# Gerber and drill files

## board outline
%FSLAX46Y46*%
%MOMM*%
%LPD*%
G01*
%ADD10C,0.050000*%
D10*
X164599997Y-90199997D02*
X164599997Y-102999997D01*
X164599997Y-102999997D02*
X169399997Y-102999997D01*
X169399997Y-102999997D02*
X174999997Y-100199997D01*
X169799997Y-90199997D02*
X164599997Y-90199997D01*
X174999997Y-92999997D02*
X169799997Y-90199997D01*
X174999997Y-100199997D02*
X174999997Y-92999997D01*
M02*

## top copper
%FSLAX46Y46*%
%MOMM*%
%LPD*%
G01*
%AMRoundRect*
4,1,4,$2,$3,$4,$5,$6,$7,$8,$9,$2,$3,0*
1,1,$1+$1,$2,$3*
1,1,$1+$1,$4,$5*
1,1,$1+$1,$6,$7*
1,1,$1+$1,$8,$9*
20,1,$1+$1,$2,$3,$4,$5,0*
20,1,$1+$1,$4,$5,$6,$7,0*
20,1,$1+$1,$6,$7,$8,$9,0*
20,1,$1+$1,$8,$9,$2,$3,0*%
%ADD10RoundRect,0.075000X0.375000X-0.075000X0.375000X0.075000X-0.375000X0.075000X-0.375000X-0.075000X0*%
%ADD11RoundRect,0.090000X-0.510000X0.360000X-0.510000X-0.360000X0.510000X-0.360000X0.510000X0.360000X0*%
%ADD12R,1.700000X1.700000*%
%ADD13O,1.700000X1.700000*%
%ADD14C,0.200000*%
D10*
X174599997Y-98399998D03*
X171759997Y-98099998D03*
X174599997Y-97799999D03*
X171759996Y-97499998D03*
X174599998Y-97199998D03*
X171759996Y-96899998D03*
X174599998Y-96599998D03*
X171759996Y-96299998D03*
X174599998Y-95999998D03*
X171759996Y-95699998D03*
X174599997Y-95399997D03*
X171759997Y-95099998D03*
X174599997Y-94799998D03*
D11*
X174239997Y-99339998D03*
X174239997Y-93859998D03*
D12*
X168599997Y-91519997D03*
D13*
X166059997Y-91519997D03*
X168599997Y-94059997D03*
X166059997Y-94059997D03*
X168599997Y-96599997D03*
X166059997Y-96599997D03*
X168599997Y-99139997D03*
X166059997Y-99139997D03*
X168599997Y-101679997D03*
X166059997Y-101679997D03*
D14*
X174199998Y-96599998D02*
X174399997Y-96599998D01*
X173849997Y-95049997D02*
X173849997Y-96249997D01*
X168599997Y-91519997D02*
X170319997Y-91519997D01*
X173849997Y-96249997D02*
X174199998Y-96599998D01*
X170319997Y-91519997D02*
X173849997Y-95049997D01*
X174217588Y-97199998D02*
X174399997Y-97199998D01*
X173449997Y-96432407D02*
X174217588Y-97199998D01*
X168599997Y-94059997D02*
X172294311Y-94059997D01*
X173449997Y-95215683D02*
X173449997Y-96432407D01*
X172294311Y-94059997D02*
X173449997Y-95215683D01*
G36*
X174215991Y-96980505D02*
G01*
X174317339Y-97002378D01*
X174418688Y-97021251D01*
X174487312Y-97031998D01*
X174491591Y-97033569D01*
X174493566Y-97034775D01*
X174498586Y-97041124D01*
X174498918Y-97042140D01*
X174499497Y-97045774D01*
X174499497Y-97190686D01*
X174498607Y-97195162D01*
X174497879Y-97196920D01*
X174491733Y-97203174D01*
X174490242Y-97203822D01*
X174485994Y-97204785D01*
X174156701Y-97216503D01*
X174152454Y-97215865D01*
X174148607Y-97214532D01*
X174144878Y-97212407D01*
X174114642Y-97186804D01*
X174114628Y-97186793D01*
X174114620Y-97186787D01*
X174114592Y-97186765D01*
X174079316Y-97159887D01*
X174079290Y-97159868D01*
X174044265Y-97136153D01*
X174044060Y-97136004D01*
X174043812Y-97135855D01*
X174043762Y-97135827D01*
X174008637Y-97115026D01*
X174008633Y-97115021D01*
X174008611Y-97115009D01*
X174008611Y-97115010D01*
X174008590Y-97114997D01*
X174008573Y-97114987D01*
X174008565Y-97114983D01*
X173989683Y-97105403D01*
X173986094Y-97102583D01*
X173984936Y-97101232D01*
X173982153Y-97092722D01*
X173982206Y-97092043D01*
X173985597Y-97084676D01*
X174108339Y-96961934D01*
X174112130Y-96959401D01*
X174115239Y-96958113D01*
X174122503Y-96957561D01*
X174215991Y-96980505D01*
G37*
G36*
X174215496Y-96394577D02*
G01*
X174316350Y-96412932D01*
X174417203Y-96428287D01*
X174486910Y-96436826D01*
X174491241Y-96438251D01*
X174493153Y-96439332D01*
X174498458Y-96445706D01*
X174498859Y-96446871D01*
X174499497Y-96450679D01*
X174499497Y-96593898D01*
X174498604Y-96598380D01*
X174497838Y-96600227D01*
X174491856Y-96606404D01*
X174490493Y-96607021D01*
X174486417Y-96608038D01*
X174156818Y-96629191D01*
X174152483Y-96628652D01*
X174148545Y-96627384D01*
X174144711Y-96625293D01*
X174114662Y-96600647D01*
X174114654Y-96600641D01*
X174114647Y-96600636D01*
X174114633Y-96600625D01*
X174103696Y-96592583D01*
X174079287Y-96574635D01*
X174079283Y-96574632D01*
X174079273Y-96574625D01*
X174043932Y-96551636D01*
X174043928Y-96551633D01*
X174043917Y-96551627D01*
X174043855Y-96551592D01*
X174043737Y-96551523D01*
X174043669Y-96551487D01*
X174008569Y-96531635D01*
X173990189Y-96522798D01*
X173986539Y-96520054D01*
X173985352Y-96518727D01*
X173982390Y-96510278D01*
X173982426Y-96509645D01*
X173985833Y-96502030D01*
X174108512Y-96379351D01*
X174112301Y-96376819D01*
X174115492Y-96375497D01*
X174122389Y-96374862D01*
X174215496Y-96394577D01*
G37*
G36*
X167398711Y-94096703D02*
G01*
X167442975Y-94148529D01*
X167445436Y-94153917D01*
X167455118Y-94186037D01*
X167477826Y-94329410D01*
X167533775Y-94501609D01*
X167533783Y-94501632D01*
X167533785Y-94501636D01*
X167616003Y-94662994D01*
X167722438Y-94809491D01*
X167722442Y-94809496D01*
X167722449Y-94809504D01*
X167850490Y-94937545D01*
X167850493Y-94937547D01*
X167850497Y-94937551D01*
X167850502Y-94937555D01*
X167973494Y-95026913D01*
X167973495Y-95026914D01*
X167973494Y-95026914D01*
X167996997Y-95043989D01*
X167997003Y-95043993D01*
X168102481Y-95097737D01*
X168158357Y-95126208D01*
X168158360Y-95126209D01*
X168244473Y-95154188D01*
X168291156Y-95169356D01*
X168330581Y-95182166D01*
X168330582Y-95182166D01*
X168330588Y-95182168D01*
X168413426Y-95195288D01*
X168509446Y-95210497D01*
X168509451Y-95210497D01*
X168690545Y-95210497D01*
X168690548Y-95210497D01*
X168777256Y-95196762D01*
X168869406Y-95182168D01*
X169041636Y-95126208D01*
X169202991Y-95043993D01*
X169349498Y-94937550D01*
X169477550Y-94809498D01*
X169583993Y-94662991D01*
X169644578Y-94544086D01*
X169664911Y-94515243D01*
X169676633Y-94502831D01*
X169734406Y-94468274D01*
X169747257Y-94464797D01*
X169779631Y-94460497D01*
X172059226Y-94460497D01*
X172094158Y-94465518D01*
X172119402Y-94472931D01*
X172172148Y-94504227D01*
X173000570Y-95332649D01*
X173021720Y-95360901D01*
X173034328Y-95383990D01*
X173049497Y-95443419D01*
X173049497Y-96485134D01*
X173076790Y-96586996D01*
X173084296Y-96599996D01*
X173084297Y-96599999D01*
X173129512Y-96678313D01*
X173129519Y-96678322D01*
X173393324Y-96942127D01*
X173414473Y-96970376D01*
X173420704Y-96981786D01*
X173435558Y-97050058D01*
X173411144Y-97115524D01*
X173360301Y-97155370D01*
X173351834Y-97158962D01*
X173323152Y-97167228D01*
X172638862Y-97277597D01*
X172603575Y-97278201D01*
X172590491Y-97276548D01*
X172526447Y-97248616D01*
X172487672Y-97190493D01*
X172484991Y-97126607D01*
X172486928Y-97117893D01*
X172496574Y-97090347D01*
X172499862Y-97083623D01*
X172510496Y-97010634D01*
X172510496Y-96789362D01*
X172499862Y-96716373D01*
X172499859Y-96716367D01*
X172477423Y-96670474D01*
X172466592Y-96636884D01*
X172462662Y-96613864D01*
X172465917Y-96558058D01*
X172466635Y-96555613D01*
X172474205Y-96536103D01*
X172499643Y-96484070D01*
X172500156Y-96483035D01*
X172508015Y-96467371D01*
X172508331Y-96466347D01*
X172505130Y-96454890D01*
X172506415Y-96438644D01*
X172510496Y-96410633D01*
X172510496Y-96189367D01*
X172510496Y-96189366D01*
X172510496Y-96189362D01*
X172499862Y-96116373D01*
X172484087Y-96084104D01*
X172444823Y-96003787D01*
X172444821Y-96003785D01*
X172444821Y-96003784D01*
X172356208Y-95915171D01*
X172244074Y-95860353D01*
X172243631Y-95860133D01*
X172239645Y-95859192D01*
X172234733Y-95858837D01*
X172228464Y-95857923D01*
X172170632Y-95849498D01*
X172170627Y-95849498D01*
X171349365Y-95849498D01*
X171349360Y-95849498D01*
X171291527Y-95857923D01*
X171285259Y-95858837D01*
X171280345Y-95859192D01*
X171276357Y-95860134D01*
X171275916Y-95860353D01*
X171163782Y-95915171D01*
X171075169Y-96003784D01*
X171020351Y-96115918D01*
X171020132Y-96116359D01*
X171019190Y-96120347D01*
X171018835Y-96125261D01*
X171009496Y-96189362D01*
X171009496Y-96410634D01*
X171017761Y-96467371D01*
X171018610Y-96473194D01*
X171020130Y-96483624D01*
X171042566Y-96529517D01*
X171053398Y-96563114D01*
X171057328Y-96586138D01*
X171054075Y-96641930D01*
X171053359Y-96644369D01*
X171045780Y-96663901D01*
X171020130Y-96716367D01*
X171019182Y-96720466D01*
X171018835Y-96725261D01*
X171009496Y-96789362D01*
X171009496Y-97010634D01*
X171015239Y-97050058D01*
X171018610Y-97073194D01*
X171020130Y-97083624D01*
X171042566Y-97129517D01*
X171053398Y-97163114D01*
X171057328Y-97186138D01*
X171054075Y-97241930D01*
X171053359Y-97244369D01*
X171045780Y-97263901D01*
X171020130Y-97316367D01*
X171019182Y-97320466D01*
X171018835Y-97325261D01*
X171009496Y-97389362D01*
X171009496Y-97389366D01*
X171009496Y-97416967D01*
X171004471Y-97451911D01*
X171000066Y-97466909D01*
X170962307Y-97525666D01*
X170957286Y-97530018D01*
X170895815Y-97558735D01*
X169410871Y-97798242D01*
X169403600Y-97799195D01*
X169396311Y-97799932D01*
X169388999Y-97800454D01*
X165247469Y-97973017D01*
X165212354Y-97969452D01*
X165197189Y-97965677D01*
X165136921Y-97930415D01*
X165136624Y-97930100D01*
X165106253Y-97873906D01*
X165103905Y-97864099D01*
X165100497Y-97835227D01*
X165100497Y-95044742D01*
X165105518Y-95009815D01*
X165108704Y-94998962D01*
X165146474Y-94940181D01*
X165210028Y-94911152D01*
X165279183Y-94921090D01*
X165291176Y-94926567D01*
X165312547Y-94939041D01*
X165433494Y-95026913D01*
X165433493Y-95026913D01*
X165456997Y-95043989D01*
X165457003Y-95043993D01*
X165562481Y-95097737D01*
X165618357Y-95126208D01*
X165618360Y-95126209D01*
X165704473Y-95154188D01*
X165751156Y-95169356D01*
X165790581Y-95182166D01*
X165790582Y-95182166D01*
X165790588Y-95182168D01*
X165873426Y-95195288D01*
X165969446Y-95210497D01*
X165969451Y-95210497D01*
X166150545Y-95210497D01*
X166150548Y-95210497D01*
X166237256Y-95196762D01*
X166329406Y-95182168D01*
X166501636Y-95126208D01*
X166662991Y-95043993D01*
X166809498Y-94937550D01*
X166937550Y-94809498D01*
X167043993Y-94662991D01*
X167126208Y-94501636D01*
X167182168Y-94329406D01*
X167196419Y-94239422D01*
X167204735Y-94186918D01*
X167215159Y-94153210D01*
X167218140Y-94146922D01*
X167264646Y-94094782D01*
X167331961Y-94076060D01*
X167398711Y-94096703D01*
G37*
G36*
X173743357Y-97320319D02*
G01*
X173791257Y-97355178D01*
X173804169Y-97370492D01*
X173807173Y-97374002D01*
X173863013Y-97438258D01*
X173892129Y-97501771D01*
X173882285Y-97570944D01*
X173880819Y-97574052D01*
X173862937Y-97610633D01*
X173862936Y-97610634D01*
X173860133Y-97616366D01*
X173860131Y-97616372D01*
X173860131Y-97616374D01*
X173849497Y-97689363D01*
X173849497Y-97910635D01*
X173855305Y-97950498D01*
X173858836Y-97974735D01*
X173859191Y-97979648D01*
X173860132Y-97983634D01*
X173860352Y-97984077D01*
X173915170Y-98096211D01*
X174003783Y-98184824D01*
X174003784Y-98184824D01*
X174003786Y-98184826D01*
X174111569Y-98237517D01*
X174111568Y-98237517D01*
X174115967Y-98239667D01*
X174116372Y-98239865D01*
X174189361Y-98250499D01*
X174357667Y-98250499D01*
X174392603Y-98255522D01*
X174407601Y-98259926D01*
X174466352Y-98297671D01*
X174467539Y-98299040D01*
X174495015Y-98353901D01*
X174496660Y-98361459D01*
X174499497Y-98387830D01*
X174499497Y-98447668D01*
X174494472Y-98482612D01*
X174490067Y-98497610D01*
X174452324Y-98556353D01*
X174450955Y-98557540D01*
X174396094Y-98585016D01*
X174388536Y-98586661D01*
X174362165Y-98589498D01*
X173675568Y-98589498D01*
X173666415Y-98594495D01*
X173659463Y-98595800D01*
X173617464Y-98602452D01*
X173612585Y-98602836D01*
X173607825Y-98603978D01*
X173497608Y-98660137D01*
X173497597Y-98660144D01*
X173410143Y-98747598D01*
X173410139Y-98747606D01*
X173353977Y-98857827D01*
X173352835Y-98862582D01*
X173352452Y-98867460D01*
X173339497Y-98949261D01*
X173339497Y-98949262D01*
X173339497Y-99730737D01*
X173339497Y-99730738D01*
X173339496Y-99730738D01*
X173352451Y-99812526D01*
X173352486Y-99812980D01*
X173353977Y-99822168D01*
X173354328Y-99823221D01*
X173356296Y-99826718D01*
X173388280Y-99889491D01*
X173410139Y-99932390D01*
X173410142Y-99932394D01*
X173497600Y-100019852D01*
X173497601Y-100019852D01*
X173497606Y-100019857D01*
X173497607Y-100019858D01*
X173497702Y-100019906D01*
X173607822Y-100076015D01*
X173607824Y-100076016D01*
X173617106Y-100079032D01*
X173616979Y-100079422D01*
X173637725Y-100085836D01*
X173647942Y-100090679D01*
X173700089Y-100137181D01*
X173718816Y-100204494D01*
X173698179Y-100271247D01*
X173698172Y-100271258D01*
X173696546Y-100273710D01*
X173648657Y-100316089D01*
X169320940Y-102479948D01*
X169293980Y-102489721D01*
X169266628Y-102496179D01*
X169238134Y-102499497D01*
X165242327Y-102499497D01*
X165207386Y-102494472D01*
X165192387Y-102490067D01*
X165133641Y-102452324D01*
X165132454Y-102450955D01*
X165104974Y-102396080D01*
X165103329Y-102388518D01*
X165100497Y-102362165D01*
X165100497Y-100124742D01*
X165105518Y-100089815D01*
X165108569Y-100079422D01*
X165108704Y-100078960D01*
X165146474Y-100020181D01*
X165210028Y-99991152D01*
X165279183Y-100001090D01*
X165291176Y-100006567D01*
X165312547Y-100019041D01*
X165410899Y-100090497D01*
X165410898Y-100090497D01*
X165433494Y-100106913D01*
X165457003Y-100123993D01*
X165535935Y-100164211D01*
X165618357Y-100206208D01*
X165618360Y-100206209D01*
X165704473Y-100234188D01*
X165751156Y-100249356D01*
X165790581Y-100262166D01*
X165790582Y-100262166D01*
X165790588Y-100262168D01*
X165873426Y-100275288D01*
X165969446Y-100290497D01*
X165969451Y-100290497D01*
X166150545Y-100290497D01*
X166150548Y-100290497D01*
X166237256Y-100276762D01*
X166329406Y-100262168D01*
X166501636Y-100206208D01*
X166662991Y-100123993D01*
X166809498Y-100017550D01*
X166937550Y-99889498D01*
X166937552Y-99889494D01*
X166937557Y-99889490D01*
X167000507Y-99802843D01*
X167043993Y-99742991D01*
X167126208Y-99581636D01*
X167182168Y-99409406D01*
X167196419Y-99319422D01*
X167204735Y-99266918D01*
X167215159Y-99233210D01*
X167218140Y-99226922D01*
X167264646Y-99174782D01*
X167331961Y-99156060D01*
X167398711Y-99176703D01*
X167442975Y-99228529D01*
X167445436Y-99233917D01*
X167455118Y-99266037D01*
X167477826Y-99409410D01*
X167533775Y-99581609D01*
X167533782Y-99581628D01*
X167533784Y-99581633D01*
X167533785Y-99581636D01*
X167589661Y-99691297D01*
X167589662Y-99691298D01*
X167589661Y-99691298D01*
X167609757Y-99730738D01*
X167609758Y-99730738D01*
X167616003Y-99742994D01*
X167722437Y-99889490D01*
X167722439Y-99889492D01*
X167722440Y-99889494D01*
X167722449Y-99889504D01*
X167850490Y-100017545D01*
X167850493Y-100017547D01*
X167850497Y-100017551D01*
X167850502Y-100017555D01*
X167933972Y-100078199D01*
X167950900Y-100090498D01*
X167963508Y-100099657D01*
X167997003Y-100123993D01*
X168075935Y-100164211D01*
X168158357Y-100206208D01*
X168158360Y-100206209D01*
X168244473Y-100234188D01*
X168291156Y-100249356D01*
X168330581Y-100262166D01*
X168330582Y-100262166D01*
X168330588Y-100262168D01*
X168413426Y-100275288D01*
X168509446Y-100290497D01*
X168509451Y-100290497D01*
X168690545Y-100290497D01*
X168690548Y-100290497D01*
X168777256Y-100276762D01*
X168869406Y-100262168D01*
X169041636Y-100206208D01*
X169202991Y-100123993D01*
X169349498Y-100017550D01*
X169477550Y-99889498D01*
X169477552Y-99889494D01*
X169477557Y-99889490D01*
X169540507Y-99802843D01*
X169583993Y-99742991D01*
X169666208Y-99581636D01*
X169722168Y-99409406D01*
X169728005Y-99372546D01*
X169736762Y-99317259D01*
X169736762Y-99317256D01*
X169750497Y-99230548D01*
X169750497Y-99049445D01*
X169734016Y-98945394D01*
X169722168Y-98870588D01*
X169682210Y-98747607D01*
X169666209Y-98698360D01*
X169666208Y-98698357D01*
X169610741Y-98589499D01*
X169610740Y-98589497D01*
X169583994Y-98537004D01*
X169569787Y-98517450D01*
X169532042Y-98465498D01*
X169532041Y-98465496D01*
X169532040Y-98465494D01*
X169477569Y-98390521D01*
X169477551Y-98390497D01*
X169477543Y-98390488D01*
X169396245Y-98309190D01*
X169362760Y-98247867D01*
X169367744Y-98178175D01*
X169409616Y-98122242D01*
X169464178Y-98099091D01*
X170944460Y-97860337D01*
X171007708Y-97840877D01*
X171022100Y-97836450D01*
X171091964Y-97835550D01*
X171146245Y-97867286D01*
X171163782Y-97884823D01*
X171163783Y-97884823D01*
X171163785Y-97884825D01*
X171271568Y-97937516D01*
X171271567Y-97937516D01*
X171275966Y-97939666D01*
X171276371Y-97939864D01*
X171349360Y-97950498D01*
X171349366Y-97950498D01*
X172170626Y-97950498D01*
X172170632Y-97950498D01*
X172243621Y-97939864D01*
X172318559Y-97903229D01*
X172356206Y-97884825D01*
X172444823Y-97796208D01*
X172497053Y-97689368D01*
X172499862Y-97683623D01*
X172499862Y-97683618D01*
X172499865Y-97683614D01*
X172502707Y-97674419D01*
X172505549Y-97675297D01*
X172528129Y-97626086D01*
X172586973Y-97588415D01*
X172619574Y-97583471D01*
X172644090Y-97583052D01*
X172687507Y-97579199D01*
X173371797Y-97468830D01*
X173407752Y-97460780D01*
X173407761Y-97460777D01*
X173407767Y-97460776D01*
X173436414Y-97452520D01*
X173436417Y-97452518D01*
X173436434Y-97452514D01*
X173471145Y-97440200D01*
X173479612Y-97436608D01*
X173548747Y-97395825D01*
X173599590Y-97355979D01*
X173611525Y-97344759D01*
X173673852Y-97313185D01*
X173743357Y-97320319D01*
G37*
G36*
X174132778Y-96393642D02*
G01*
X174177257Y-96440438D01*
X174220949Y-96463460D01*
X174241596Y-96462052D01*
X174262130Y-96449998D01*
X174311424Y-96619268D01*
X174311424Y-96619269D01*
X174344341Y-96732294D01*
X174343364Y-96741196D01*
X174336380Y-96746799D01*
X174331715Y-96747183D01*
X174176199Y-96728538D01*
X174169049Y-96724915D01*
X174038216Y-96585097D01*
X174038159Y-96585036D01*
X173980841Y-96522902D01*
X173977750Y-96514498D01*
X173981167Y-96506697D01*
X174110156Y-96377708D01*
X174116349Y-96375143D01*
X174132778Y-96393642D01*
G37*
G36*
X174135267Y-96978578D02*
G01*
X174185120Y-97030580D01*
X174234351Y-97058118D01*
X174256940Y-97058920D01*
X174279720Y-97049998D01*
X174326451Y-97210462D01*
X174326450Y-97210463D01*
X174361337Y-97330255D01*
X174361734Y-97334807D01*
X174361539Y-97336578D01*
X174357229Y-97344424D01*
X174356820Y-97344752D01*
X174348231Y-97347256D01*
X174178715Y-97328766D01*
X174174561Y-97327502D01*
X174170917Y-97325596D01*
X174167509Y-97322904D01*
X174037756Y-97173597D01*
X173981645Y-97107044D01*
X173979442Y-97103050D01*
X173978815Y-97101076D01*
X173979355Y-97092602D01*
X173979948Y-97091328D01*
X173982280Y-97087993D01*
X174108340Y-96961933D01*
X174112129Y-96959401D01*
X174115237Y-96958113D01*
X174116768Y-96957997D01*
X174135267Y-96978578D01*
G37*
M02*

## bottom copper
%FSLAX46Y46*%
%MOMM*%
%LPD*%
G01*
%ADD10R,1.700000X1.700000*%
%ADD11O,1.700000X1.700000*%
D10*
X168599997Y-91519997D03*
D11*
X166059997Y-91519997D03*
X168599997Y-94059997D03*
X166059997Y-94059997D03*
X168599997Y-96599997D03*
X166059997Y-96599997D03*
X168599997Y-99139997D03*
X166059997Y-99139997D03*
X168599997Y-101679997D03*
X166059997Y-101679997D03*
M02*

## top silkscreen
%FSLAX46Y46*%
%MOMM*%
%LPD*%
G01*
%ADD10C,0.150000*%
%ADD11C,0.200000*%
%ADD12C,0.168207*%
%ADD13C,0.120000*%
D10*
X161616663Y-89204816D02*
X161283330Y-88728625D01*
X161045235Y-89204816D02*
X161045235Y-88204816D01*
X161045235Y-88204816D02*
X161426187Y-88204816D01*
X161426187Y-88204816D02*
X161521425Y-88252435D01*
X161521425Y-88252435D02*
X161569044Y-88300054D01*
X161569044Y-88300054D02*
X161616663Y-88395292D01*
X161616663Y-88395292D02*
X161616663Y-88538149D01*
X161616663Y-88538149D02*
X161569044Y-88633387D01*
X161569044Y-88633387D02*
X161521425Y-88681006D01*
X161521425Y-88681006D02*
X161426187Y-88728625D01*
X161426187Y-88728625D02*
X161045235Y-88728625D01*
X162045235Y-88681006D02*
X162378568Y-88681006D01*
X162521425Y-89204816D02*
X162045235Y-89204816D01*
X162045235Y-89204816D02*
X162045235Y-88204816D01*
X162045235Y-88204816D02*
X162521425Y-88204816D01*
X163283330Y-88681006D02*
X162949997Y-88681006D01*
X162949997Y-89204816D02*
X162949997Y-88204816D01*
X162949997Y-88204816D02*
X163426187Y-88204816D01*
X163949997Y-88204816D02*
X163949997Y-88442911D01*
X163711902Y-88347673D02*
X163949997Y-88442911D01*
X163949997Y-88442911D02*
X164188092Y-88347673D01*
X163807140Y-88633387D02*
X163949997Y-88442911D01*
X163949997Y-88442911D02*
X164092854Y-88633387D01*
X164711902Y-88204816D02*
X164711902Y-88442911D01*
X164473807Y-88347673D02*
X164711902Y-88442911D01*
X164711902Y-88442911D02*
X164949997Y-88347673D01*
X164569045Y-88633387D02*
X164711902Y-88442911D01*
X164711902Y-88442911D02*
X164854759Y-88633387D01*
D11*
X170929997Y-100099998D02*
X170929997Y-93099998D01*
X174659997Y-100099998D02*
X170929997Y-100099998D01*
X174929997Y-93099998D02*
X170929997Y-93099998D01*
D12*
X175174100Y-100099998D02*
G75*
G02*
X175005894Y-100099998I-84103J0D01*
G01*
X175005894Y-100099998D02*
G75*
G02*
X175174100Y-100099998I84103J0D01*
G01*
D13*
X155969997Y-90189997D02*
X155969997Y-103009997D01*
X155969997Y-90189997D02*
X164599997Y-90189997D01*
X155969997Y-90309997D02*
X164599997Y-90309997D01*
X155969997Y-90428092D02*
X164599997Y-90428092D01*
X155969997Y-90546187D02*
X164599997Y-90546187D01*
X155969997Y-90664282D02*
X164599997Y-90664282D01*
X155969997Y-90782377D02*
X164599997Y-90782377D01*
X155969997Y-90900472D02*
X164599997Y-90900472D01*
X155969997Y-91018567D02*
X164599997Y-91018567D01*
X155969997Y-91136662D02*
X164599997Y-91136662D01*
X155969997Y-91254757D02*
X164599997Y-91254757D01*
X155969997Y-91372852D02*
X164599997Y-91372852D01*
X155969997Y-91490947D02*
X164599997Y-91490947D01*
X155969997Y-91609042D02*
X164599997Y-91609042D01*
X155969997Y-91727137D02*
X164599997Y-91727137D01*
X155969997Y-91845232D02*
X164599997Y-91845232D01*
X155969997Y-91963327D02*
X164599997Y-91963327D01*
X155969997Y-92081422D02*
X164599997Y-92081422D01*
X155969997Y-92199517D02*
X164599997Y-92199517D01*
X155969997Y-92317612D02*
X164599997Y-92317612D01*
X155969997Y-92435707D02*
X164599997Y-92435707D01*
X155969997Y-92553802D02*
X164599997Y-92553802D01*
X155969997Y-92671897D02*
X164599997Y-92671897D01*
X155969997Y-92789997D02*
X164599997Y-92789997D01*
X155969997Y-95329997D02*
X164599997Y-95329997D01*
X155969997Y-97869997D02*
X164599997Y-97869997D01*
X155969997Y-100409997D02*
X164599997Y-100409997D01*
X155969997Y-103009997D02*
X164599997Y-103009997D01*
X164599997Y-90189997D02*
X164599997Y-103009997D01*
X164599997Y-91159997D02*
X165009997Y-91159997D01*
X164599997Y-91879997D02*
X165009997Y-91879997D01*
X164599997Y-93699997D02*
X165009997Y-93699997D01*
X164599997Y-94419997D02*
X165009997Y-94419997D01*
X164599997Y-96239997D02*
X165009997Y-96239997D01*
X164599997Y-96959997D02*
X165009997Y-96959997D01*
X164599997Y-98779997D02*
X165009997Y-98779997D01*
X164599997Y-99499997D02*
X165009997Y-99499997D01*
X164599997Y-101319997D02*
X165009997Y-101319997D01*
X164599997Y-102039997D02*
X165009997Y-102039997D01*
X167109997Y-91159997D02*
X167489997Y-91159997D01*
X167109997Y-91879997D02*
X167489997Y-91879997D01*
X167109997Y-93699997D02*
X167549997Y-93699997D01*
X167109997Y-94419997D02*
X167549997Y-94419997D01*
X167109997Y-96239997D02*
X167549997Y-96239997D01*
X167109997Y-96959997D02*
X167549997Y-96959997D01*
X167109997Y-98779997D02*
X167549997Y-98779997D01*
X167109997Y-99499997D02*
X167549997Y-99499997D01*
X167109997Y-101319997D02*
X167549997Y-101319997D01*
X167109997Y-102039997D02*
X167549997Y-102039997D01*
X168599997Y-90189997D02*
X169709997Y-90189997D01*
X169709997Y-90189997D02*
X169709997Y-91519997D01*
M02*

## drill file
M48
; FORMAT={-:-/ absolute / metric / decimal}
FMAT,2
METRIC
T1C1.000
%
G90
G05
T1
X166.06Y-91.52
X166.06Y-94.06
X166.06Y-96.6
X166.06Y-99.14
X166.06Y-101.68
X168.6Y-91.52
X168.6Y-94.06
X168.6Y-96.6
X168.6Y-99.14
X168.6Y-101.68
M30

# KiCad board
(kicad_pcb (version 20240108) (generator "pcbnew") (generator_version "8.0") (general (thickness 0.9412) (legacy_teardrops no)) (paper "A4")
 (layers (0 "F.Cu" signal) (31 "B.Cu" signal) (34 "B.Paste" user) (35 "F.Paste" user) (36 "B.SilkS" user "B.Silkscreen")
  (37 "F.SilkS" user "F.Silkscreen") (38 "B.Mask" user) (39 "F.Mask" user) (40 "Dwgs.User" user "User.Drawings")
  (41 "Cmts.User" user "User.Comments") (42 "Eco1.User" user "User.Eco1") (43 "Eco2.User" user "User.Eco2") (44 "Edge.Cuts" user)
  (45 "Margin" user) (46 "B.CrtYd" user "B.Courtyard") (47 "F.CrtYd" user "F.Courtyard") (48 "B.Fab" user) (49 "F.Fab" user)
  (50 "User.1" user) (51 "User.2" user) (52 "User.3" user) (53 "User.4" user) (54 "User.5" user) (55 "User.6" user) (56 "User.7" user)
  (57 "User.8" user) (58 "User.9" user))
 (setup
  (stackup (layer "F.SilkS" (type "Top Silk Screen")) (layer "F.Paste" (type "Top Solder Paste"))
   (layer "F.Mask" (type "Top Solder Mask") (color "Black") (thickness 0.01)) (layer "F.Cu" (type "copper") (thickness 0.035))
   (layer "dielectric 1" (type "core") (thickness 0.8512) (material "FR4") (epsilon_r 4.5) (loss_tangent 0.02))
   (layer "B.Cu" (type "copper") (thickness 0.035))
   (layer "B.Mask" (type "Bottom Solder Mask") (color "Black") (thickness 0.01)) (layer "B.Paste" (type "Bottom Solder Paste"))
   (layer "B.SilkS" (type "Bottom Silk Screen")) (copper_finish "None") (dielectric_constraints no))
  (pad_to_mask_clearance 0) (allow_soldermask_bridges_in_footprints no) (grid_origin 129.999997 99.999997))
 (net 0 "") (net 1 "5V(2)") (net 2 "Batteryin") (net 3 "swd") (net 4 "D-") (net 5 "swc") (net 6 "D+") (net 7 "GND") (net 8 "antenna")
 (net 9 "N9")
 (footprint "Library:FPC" (layer "F.Cu") (at 173.179997 96.599998 90)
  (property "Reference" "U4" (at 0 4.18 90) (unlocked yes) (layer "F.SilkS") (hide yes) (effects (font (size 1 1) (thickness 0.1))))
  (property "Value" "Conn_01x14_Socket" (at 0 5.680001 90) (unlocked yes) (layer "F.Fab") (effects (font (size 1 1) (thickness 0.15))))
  (fp_line (start -3.5 -2.25) (end 3.5 -2.25) (stroke (width 0.2) (type default)) (layer "F.SilkS"))
  (fp_line (start -3.5 1.48) (end -3.5 -2.25) (stroke (width 0.2) (type default)) (layer "F.SilkS"))
  (fp_line (start 3.5 1.75) (end 3.5 -2.25) (stroke (width 0.2) (type default)) (layer "F.SilkS"))
  (fp_circle (center -3.5 1.91) (end -3.382638 1.89589) (stroke (width 0.1) (type solid)) (fill solid) (layer "F.SilkS"))
  (pad "1" smd roundrect (at -1.8 1.42 90) (size 0.3 0.9) (layers "F.Cu" "F.Paste" "F.Mask") (roundrect_rratio 0.25) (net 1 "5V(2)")
   (thermal_bridge_angle 45)
   (teardrops (best_length_ratio 0.5) (max_length 1) (best_width_ratio 1) (max_width 2) (curve_points 5) (filter_ratio 0.9) (enabled yes)
    (allow_two_segments yes) (prefer_zone_connections yes)))
  (pad "2" smd roundrect (at -1.5 -1.42 90) (size 0.3 0.9) (layers "F.Cu" "F.Paste" "F.Mask") (roundrect_rratio 0.25) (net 1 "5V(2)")
   (thermal_bridge_angle 45)
   (teardrops (best_length_ratio 0.5) (max_length 1) (best_width_ratio 1) (max_width 2) (curve_points 5) (filter_ratio 0.9) (enabled yes)
    (allow_two_segments yes) (prefer_zone_connections yes)))
  (pad "3" smd roundrect (at -1.200001 1.42 90) (size 0.3 0.9) (layers "F.Cu" "F.Paste" "F.Mask") (roundrect_rratio 0.25)
   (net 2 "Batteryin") (thermal_bridge_angle 45)
   (teardrops (best_length_ratio 0.5) (max_length 1) (best_width_ratio 1) (max_width 2) (curve_points 5) (filter_ratio 0.9) (enabled yes)
    (allow_two_segments yes) (prefer_zone_connections yes)))
  (pad "4" smd roundrect (at -0.9 -1.420001 90) (size 0.3 0.9) (layers "F.Cu" "F.Paste" "F.Mask") (roundrect_rratio 0.25)
   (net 2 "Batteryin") (thermal_bridge_angle 45)
   (teardrops (best_length_ratio 0.5) (max_length 1) (best_width_ratio 1) (max_width 2) (curve_points 5) (filter_ratio 0.9) (enabled yes)
    (allow_two_segments yes) (prefer_zone_connections yes)))
  (pad "5" smd roundrect (at -0.6 1.420001 90) (size 0.3 0.9) (layers "F.Cu" "F.Paste" "F.Mask") (roundrect_rratio 0.25) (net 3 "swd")
   (thermal_bridge_angle 45)
   (teardrops (best_length_ratio 0.5) (max_length 1) (best_width_ratio 1) (max_width 2) (curve_points 5) (filter_ratio 0.9) (enabled yes)
    (allow_two_segments yes) (prefer_zone_connections yes)))
  (pad "6" smd roundrect (at -0.3 -1.420001 90) (size 0.3 0.9) (layers "F.Cu" "F.Paste" "F.Mask") (roundrect_rratio 0.25) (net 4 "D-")
   (thermal_bridge_angle 45)
   (teardrops (best_length_ratio 0.5) (max_length 1) (best_width_ratio 1) (max_width 2) (curve_points 5) (filter_ratio 0.9) (enabled yes)
    (allow_two_segments yes) (prefer_zone_connections yes)))
  (pad "7" smd roundrect (at 0 1.420001 90) (size 0.3 0.9) (layers "F.Cu" "F.Paste" "F.Mask") (roundrect_rratio 0.25) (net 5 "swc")
   (thermal_bridge_angle 45)
   (teardrops (best_length_ratio 0.5) (max_length 1) (best_width_ratio 1) (max_width 2) (curve_points 5) (filter_ratio 0.9) (enabled yes)
    (allow_two_segments yes) (prefer_zone_connections yes)))
  (pad "8" smd roundrect (at 0.3 -1.420001 90) (size 0.3 0.9) (layers "F.Cu" "F.Paste" "F.Mask") (roundrect_rratio 0.25) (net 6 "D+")
   (thermal_bridge_angle 45)
   (teardrops (best_length_ratio 0.5) (max_length 1) (best_width_ratio 1) (max_width 2) (curve_points 5) (filter_ratio 0.9) (enabled yes)
    (allow_two_segments yes) (prefer_zone_connections yes)))
  (pad "9" smd roundrect (at 0.6 1.420001 90) (size 0.3 0.9) (layers "F.Cu" "F.Paste" "F.Mask") (roundrect_rratio 0.25) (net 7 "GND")
   (thermal_bridge_angle 45)
   (teardrops (best_length_ratio 0.5) (max_length 1) (best_width_ratio 1) (max_width 2) (curve_points 5) (filter_ratio 0.9) (enabled yes)
    (allow_two_segments yes) (prefer_zone_connections yes)))
  (pad "10" smd roundrect (at 0.9 -1.420001 90) (size 0.3 0.9) (layers "F.Cu" "F.Paste" "F.Mask") (roundrect_rratio 0.25) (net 7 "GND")
   (thermal_bridge_angle 45)
   (teardrops (best_length_ratio 0.5) (max_length 1) (best_width_ratio 1) (max_width 2) (curve_points 5) (filter_ratio 0.9) (enabled yes)
    (allow_two_segments yes) (prefer_zone_connections yes)))
  (pad "11" smd roundrect (at 1.200001 1.42 90) (size 0.3 0.9) (layers "F.Cu" "F.Paste" "F.Mask") (roundrect_rratio 0.25) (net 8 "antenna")
   (thermal_bridge_angle 45)
   (teardrops (best_length_ratio 0.5) (max_length 1) (best_width_ratio 1) (max_width 2) (curve_points 5) (filter_ratio 0.9) (enabled yes)
    (allow_two_segments yes) (prefer_zone_connections yes)))
  (pad "12" smd roundrect (at 1.5 -1.42 90) (size 0.3 0.9) (layers "F.Cu" "F.Paste" "F.Mask") (roundrect_rratio 0.25) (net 7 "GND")
   (thermal_bridge_angle 45)
   (teardrops (best_length_ratio 0.5) (max_length 1) (best_width_ratio 1) (max_width 2) (curve_points 5) (filter_ratio 0.9) (enabled yes)
    (allow_two_segments yes) (prefer_zone_connections yes)))
  (pad "13" smd roundrect (at 1.8 1.42 90) (size 0.3 0.9) (layers "F.Cu" "F.Paste" "F.Mask") (roundrect_rratio 0.25) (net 7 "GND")
   (thermal_bridge_angle 45)
   (teardrops (best_length_ratio 0.5) (max_length 1) (best_width_ratio 1) (max_width 2) (curve_points 5) (filter_ratio 0.9) (enabled yes)
    (allow_two_segments yes) (prefer_zone_connections yes)))
  (pad "14" smd roundrect (at -2.74 1.06 270) (size 0.9 1.2) (layers "F.Cu" "F.Paste" "F.Mask") (roundrect_rratio 0.1) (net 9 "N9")
   (thermal_bridge_angle 45))
  (pad "15" smd roundrect (at 2.74 1.06 270) (size 0.9 1.2) (layers "F.Cu" "F.Paste" "F.Mask") (roundrect_rratio 0.1)
   (thermal_bridge_angle 45)))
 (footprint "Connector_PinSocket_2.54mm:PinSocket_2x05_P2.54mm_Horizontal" (layer "F.Cu") (at 168.599997 91.519997)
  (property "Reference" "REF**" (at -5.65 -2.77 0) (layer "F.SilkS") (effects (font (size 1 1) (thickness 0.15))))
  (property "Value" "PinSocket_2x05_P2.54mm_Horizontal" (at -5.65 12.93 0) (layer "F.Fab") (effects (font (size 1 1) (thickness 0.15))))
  (fp_line (start -12.63 -1.33) (end -12.63 11.49) (stroke (width 0.12) (type solid)) (layer "F.SilkS"))
  (fp_line (start -12.63 -1.33) (end -4 -1.33) (stroke (width 0.12) (type solid)) (layer "F.SilkS"))
  (fp_line (start -12.63 -1.21) (end -4 -1.21) (stroke (width 0.12) (type solid)) (layer "F.SilkS"))
  (fp_line (start -12.63 -1.091905) (end -4 -1.091905) (stroke (width 0.12) (type solid)) (layer "F.SilkS"))
  (fp_line (start -12.63 -0.97381) (end -4 -0.97381) (stroke (width 0.12) (type solid)) (layer "F.SilkS"))
  (fp_line (start -12.63 -0.855715) (end -4 -0.855715) (stroke (width 0.12) (type solid)) (layer "F.SilkS"))
  (fp_line (start -12.63 -0.73762) (end -4 -0.73762) (stroke (width 0.12) (type solid)) (layer "F.SilkS"))
  (fp_line (start -12.63 -0.619525) (end -4 -0.619525) (stroke (width 0.12) (type solid)) (layer "F.SilkS"))
  (fp_line (start -12.63 -0.50143) (end -4 -0.50143) (stroke (width 0.12) (type solid)) (layer "F.SilkS"))
  (fp_line (start -12.63 -0.383335) (end -4 -0.383335) (stroke (width 0.12) (type solid)) (layer "F.SilkS"))
  (fp_line (start -12.63 -0.26524) (end -4 -0.26524) (stroke (width 0.12) (type solid)) (layer "F.SilkS"))
  (fp_line (start -12.63 -0.147145) (end -4 -0.147145) (stroke (width 0.12) (type solid)) (layer "F.SilkS"))
  (fp_line (start -12.63 -0.02905) (end -4 -0.02905) (stroke (width 0.12) (type solid)) (layer "F.SilkS"))
  (fp_line (start -12.63 0.089045) (end -4 0.089045) (stroke (width 0.12) (type solid)) (layer "F.SilkS"))
  (fp_line (start -12.63 0.20714) (end -4 0.20714) (stroke (width 0.12) (type solid)) (layer "F.SilkS"))
  (fp_line (start -12.63 0.325235) (end -4 0.325235) (stroke (width 0.12) (type solid)) (layer "F.SilkS"))
  (fp_line (start -12.63 0.44333) (end -4 0.44333) (stroke (width 0.12) (type solid)) (layer "F.SilkS"))
  (fp_line (start -12.63 0.561425) (end -4 0.561425) (stroke (width 0.12) (type solid)) (layer "F.SilkS"))
  (fp_line (start -12.63 0.67952) (end -4 0.67952) (stroke (width 0.12) (type solid)) (layer "F.SilkS"))
  (fp_line (start -12.63 0.797615) (end -4 0.797615) (stroke (width 0.12) (type solid)) (layer "F.SilkS"))
  (fp_line (start -12.63 0.91571) (end -4 0.91571) (stroke (width 0.12) (type solid)) (layer "F.SilkS"))
  (fp_line (start -12.63 1.033805) (end -4 1.033805) (stroke (width 0.12) (type solid)) (layer "F.SilkS"))
  (fp_line (start -12.63 1.1519) (end -4 1.1519) (stroke (width 0.12) (type solid)) (layer "F.SilkS"))
  (fp_line (start -12.63 1.27) (end -4 1.27) (stroke (width 0.12) (type solid)) (layer "F.SilkS"))
  (fp_line (start -12.63 3.81) (end -4 3.81) (stroke (width 0.12) (type solid)) (layer "F.SilkS"))
  (fp_line (start -12.63 6.35) (end -4 6.35) (stroke (width 0.12) (type solid)) (layer "F.SilkS"))
  (fp_line (start -12.63 8.89) (end -4 8.89) (stroke (width 0.12) (type solid)) (layer "F.SilkS"))
  (fp_line (start -12.63 11.49) (end -4 11.49) (stroke (width 0.12) (type solid)) (layer "F.SilkS"))
  (fp_line (start -4 -1.33) (end -4 11.49) (stroke (width 0.12) (type solid)) (layer "F.SilkS"))
  (fp_line (start -4 -0.36) (end -3.59 -0.36) (stroke (width 0.12) (type solid)) (layer "F.SilkS"))
  (fp_line (start -4 0.36) (end -3.59 0.36) (stroke (width 0.12) (type solid)) (layer "F.SilkS"))
  (fp_line (start -4 2.18) (end -3.59 2.18) (stroke (width 0.12) (type solid)) (layer "F.SilkS"))
  (fp_line (start -4 2.9) (end -3.59 2.9) (stroke (width 0.12) (type solid)) (layer "F.SilkS"))
  (fp_line (start -4 4.72) (end -3.59 4.72) (stroke (width 0.12) (type solid)) (layer "F.SilkS"))
  (fp_line (start -4 5.44) (end -3.59 5.44) (stroke (width 0.12) (type solid)) (layer "F.SilkS"))
  (fp_line (start -4 7.26) (end -3.59 7.26) (stroke (width 0.12) (type solid)) (layer "F.SilkS"))
  (fp_line (start -4 7.98) (end -3.59 7.98) (stroke (width 0.12) (type solid)) (layer "F.SilkS"))
  (fp_line (start -4 9.8) (end -3.59 9.8) (stroke (width 0.12) (type solid)) (layer "F.SilkS"))
  (fp_line (start -4 10.52) (end -3.59 10.52) (stroke (width 0.12) (type solid)) (layer "F.SilkS"))
  (fp_line (start -1.49 -0.36) (end -1.11 -0.36) (stroke (width 0.12) (type solid)) (layer "F.SilkS"))
  (fp_line (start -1.49 0.36) (end -1.11 0.36) (stroke (width 0.12) (type solid)) (layer "F.SilkS"))
  (fp_line (start -1.49 2.18) (end -1.05 2.18) (stroke (width 0.12) (type solid)) (layer "F.SilkS"))
  (fp_line (start -1.49 2.9) (end -1.05 2.9) (stroke (width 0.12) (type solid)) (layer "F.SilkS"))
  (fp_line (start -1.49 4.72) (end -1.05 4.72) (stroke (width 0.12) (type solid)) (layer "F.SilkS"))
  (fp_line (start -1.49 5.44) (end -1.05 5.44) (stroke (width 0.12) (type solid)) (layer "F.SilkS"))
  (fp_line (start -1.49 7.26) (end -1.05 7.26) (stroke (width 0.12) (type solid)) (layer "F.SilkS"))
  (fp_line (start -1.49 7.98) (end -1.05 7.98) (stroke (width 0.12) (type solid)) (layer "F.SilkS"))
  (fp_line (start -1.49 9.8) (end -1.05 9.8) (stroke (width 0.12) (type solid)) (layer "F.SilkS"))
  (fp_line (start -1.49 10.52) (end -1.05 10.52) (stroke (width 0.12) (type solid)) (layer "F.SilkS"))
  (fp_line (start 0 -1.33) (end 1.11 -1.33) (stroke (width 0.12) (type solid)) (layer "F.SilkS"))
  (fp_line (start 1.11 -1.33) (end 1.11 0) (stroke (width 0.12) (type solid)) (layer "F.SilkS"))
  (pad "1" thru_hole rect (at 0 0) (size 1.7 1.7) (drill 1) (layers "*.Cu" "*.Mask") (remove_unused_layers no) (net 5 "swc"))
  (pad "2" thru_hole oval (at -2.54 0) (size 1.7 1.7) (drill 1) (layers "*.Cu" "*.Mask") (remove_unused_layers no))
  (pad "3" thru_hole oval (at 0 2.54) (size 1.7 1.7) (drill 1) (layers "*.Cu" "*.Mask") (remove_unused_layers no) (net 3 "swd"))
  (pad "4" thru_hole oval (at -2.54 2.54) (size 1.7 1.7) (drill 1) (layers "*.Cu" "*.Mask") (remove_unused_layers no))
  (pad "5" thru_hole oval (at 0 5.08) (size 1.7 1.7) (drill 1) (layers "*.Cu" "*.Mask") (remove_unused_layers no) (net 7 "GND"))
  (pad "6" thru_hole oval (at -2.54 5.08) (size 1.7 1.7) (drill 1) (layers "*.Cu" "*.Mask") (remove_unused_layers no) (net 7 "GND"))
  (pad "7" thru_hole oval (at 0 7.62) (size 1.7 1.7) (drill 1) (layers "*.Cu" "*.Mask") (remove_unused_layers no))
  (pad "8" thru_hole oval (at -2.54 7.62) (size 1.7 1.7) (drill 1) (layers "*.Cu" "*.Mask") (remove_unused_layers no))
  (pad "9" thru_hole oval (at 0 10.16) (size 1.7 1.7) (drill 1) (layers "*.Cu" "*.Mask") (remove_unused_layers no) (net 1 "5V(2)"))
  (pad "10" thru_hole oval (at -2.54 10.16) (size 1.7 1.7) (drill 1) (layers "*.Cu" "*.Mask") (remove_unused_layers no) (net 1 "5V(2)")))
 (gr_line (start 164.599997 90.199997) (end 164.599997 102.999997) (stroke (width 0.05) (type default)) (layer "Edge.Cuts"))
 (gr_line (start 164.599997 102.999997) (end 169.399997 102.999997) (stroke (width 0.05) (type default)) (layer "Edge.Cuts"))
 (gr_line (start 169.399997 102.999997) (end 174.999997 100.199997) (stroke (width 0.05) (type default)) (layer "Edge.Cuts"))
 (gr_line (start 169.799997 90.199997) (end 164.599997 90.199997) (stroke (width 0.05) (type default)) (layer "Edge.Cuts"))
 (gr_line (start 174.999997 92.999997) (end 169.799997 90.199997) (stroke (width 0.05) (type default)) (layer "Edge.Cuts"))
 (gr_line (start 174.999997 100.199997) (end 174.999997 92.999997) (stroke (width 0.05) (type default)) (layer "Edge.Cuts"))
 (segment (start 174.199998 96.599998) (end 174.399997 96.599998) (width 0.2) (layer "F.Cu") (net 5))
 (segment (start 173.849997 95.049997) (end 173.849997 96.249997) (width 0.2) (layer "F.Cu") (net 5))
 (segment (start 168.599997 91.519997) (end 170.319997 91.519997) (width 0.2) (layer "F.Cu") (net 5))
 (segment (start 173.849997 96.249997) (end 174.199998 96.599998) (width 0.2) (layer "F.Cu") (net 5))
 (segment (start 170.319997 91.519997) (end 173.849997 95.049997) (width 0.2) (layer "F.Cu") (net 5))
 (segment (start 174.217588 97.199998) (end 174.399997 97.199998) (width 0.2) (layer "F.Cu") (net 3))
 (segment (start 173.449997 96.432407) (end 174.217588 97.199998) (width 0.2) (layer "F.Cu") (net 3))
 (segment (start 168.599997 94.059997) (end 172.294311 94.059997) (width 0.2) (layer "F.Cu") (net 3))
 (segment (start 173.449997 95.215683) (end 173.449997 96.432407) (width 0.2) (layer "F.Cu") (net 3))
 (segment (start 172.294311 94.059997) (end 173.449997 95.215683) (width 0.2) (layer "F.Cu") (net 3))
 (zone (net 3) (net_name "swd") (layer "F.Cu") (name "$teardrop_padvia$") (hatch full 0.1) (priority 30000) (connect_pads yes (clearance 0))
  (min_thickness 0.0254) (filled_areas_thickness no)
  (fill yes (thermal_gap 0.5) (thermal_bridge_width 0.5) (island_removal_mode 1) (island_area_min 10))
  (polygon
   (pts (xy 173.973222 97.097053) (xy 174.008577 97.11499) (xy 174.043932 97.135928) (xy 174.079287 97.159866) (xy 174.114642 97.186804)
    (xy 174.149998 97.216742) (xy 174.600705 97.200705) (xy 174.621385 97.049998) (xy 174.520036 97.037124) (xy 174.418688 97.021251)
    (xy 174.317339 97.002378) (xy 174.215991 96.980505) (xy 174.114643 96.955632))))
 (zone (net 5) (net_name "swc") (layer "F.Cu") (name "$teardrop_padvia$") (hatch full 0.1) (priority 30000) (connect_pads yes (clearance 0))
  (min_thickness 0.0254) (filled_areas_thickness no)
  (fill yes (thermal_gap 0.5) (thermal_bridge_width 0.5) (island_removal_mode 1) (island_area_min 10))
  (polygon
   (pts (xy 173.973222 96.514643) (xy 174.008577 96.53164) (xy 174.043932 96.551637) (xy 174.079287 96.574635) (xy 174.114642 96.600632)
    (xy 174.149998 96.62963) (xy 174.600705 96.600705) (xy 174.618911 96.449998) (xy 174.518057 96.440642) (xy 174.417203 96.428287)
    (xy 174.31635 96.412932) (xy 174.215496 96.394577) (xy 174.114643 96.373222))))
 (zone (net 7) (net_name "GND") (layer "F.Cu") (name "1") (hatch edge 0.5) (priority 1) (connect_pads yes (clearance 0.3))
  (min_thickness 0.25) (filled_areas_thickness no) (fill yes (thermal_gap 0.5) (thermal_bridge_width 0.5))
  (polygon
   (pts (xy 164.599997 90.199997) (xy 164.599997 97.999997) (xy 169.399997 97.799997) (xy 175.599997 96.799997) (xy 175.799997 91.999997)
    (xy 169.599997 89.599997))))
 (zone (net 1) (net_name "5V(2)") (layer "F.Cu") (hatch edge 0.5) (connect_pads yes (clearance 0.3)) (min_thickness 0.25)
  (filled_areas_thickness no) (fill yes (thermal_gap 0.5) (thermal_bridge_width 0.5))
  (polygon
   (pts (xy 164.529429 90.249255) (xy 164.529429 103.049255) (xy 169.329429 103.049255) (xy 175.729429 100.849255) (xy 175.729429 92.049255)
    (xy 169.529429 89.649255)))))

